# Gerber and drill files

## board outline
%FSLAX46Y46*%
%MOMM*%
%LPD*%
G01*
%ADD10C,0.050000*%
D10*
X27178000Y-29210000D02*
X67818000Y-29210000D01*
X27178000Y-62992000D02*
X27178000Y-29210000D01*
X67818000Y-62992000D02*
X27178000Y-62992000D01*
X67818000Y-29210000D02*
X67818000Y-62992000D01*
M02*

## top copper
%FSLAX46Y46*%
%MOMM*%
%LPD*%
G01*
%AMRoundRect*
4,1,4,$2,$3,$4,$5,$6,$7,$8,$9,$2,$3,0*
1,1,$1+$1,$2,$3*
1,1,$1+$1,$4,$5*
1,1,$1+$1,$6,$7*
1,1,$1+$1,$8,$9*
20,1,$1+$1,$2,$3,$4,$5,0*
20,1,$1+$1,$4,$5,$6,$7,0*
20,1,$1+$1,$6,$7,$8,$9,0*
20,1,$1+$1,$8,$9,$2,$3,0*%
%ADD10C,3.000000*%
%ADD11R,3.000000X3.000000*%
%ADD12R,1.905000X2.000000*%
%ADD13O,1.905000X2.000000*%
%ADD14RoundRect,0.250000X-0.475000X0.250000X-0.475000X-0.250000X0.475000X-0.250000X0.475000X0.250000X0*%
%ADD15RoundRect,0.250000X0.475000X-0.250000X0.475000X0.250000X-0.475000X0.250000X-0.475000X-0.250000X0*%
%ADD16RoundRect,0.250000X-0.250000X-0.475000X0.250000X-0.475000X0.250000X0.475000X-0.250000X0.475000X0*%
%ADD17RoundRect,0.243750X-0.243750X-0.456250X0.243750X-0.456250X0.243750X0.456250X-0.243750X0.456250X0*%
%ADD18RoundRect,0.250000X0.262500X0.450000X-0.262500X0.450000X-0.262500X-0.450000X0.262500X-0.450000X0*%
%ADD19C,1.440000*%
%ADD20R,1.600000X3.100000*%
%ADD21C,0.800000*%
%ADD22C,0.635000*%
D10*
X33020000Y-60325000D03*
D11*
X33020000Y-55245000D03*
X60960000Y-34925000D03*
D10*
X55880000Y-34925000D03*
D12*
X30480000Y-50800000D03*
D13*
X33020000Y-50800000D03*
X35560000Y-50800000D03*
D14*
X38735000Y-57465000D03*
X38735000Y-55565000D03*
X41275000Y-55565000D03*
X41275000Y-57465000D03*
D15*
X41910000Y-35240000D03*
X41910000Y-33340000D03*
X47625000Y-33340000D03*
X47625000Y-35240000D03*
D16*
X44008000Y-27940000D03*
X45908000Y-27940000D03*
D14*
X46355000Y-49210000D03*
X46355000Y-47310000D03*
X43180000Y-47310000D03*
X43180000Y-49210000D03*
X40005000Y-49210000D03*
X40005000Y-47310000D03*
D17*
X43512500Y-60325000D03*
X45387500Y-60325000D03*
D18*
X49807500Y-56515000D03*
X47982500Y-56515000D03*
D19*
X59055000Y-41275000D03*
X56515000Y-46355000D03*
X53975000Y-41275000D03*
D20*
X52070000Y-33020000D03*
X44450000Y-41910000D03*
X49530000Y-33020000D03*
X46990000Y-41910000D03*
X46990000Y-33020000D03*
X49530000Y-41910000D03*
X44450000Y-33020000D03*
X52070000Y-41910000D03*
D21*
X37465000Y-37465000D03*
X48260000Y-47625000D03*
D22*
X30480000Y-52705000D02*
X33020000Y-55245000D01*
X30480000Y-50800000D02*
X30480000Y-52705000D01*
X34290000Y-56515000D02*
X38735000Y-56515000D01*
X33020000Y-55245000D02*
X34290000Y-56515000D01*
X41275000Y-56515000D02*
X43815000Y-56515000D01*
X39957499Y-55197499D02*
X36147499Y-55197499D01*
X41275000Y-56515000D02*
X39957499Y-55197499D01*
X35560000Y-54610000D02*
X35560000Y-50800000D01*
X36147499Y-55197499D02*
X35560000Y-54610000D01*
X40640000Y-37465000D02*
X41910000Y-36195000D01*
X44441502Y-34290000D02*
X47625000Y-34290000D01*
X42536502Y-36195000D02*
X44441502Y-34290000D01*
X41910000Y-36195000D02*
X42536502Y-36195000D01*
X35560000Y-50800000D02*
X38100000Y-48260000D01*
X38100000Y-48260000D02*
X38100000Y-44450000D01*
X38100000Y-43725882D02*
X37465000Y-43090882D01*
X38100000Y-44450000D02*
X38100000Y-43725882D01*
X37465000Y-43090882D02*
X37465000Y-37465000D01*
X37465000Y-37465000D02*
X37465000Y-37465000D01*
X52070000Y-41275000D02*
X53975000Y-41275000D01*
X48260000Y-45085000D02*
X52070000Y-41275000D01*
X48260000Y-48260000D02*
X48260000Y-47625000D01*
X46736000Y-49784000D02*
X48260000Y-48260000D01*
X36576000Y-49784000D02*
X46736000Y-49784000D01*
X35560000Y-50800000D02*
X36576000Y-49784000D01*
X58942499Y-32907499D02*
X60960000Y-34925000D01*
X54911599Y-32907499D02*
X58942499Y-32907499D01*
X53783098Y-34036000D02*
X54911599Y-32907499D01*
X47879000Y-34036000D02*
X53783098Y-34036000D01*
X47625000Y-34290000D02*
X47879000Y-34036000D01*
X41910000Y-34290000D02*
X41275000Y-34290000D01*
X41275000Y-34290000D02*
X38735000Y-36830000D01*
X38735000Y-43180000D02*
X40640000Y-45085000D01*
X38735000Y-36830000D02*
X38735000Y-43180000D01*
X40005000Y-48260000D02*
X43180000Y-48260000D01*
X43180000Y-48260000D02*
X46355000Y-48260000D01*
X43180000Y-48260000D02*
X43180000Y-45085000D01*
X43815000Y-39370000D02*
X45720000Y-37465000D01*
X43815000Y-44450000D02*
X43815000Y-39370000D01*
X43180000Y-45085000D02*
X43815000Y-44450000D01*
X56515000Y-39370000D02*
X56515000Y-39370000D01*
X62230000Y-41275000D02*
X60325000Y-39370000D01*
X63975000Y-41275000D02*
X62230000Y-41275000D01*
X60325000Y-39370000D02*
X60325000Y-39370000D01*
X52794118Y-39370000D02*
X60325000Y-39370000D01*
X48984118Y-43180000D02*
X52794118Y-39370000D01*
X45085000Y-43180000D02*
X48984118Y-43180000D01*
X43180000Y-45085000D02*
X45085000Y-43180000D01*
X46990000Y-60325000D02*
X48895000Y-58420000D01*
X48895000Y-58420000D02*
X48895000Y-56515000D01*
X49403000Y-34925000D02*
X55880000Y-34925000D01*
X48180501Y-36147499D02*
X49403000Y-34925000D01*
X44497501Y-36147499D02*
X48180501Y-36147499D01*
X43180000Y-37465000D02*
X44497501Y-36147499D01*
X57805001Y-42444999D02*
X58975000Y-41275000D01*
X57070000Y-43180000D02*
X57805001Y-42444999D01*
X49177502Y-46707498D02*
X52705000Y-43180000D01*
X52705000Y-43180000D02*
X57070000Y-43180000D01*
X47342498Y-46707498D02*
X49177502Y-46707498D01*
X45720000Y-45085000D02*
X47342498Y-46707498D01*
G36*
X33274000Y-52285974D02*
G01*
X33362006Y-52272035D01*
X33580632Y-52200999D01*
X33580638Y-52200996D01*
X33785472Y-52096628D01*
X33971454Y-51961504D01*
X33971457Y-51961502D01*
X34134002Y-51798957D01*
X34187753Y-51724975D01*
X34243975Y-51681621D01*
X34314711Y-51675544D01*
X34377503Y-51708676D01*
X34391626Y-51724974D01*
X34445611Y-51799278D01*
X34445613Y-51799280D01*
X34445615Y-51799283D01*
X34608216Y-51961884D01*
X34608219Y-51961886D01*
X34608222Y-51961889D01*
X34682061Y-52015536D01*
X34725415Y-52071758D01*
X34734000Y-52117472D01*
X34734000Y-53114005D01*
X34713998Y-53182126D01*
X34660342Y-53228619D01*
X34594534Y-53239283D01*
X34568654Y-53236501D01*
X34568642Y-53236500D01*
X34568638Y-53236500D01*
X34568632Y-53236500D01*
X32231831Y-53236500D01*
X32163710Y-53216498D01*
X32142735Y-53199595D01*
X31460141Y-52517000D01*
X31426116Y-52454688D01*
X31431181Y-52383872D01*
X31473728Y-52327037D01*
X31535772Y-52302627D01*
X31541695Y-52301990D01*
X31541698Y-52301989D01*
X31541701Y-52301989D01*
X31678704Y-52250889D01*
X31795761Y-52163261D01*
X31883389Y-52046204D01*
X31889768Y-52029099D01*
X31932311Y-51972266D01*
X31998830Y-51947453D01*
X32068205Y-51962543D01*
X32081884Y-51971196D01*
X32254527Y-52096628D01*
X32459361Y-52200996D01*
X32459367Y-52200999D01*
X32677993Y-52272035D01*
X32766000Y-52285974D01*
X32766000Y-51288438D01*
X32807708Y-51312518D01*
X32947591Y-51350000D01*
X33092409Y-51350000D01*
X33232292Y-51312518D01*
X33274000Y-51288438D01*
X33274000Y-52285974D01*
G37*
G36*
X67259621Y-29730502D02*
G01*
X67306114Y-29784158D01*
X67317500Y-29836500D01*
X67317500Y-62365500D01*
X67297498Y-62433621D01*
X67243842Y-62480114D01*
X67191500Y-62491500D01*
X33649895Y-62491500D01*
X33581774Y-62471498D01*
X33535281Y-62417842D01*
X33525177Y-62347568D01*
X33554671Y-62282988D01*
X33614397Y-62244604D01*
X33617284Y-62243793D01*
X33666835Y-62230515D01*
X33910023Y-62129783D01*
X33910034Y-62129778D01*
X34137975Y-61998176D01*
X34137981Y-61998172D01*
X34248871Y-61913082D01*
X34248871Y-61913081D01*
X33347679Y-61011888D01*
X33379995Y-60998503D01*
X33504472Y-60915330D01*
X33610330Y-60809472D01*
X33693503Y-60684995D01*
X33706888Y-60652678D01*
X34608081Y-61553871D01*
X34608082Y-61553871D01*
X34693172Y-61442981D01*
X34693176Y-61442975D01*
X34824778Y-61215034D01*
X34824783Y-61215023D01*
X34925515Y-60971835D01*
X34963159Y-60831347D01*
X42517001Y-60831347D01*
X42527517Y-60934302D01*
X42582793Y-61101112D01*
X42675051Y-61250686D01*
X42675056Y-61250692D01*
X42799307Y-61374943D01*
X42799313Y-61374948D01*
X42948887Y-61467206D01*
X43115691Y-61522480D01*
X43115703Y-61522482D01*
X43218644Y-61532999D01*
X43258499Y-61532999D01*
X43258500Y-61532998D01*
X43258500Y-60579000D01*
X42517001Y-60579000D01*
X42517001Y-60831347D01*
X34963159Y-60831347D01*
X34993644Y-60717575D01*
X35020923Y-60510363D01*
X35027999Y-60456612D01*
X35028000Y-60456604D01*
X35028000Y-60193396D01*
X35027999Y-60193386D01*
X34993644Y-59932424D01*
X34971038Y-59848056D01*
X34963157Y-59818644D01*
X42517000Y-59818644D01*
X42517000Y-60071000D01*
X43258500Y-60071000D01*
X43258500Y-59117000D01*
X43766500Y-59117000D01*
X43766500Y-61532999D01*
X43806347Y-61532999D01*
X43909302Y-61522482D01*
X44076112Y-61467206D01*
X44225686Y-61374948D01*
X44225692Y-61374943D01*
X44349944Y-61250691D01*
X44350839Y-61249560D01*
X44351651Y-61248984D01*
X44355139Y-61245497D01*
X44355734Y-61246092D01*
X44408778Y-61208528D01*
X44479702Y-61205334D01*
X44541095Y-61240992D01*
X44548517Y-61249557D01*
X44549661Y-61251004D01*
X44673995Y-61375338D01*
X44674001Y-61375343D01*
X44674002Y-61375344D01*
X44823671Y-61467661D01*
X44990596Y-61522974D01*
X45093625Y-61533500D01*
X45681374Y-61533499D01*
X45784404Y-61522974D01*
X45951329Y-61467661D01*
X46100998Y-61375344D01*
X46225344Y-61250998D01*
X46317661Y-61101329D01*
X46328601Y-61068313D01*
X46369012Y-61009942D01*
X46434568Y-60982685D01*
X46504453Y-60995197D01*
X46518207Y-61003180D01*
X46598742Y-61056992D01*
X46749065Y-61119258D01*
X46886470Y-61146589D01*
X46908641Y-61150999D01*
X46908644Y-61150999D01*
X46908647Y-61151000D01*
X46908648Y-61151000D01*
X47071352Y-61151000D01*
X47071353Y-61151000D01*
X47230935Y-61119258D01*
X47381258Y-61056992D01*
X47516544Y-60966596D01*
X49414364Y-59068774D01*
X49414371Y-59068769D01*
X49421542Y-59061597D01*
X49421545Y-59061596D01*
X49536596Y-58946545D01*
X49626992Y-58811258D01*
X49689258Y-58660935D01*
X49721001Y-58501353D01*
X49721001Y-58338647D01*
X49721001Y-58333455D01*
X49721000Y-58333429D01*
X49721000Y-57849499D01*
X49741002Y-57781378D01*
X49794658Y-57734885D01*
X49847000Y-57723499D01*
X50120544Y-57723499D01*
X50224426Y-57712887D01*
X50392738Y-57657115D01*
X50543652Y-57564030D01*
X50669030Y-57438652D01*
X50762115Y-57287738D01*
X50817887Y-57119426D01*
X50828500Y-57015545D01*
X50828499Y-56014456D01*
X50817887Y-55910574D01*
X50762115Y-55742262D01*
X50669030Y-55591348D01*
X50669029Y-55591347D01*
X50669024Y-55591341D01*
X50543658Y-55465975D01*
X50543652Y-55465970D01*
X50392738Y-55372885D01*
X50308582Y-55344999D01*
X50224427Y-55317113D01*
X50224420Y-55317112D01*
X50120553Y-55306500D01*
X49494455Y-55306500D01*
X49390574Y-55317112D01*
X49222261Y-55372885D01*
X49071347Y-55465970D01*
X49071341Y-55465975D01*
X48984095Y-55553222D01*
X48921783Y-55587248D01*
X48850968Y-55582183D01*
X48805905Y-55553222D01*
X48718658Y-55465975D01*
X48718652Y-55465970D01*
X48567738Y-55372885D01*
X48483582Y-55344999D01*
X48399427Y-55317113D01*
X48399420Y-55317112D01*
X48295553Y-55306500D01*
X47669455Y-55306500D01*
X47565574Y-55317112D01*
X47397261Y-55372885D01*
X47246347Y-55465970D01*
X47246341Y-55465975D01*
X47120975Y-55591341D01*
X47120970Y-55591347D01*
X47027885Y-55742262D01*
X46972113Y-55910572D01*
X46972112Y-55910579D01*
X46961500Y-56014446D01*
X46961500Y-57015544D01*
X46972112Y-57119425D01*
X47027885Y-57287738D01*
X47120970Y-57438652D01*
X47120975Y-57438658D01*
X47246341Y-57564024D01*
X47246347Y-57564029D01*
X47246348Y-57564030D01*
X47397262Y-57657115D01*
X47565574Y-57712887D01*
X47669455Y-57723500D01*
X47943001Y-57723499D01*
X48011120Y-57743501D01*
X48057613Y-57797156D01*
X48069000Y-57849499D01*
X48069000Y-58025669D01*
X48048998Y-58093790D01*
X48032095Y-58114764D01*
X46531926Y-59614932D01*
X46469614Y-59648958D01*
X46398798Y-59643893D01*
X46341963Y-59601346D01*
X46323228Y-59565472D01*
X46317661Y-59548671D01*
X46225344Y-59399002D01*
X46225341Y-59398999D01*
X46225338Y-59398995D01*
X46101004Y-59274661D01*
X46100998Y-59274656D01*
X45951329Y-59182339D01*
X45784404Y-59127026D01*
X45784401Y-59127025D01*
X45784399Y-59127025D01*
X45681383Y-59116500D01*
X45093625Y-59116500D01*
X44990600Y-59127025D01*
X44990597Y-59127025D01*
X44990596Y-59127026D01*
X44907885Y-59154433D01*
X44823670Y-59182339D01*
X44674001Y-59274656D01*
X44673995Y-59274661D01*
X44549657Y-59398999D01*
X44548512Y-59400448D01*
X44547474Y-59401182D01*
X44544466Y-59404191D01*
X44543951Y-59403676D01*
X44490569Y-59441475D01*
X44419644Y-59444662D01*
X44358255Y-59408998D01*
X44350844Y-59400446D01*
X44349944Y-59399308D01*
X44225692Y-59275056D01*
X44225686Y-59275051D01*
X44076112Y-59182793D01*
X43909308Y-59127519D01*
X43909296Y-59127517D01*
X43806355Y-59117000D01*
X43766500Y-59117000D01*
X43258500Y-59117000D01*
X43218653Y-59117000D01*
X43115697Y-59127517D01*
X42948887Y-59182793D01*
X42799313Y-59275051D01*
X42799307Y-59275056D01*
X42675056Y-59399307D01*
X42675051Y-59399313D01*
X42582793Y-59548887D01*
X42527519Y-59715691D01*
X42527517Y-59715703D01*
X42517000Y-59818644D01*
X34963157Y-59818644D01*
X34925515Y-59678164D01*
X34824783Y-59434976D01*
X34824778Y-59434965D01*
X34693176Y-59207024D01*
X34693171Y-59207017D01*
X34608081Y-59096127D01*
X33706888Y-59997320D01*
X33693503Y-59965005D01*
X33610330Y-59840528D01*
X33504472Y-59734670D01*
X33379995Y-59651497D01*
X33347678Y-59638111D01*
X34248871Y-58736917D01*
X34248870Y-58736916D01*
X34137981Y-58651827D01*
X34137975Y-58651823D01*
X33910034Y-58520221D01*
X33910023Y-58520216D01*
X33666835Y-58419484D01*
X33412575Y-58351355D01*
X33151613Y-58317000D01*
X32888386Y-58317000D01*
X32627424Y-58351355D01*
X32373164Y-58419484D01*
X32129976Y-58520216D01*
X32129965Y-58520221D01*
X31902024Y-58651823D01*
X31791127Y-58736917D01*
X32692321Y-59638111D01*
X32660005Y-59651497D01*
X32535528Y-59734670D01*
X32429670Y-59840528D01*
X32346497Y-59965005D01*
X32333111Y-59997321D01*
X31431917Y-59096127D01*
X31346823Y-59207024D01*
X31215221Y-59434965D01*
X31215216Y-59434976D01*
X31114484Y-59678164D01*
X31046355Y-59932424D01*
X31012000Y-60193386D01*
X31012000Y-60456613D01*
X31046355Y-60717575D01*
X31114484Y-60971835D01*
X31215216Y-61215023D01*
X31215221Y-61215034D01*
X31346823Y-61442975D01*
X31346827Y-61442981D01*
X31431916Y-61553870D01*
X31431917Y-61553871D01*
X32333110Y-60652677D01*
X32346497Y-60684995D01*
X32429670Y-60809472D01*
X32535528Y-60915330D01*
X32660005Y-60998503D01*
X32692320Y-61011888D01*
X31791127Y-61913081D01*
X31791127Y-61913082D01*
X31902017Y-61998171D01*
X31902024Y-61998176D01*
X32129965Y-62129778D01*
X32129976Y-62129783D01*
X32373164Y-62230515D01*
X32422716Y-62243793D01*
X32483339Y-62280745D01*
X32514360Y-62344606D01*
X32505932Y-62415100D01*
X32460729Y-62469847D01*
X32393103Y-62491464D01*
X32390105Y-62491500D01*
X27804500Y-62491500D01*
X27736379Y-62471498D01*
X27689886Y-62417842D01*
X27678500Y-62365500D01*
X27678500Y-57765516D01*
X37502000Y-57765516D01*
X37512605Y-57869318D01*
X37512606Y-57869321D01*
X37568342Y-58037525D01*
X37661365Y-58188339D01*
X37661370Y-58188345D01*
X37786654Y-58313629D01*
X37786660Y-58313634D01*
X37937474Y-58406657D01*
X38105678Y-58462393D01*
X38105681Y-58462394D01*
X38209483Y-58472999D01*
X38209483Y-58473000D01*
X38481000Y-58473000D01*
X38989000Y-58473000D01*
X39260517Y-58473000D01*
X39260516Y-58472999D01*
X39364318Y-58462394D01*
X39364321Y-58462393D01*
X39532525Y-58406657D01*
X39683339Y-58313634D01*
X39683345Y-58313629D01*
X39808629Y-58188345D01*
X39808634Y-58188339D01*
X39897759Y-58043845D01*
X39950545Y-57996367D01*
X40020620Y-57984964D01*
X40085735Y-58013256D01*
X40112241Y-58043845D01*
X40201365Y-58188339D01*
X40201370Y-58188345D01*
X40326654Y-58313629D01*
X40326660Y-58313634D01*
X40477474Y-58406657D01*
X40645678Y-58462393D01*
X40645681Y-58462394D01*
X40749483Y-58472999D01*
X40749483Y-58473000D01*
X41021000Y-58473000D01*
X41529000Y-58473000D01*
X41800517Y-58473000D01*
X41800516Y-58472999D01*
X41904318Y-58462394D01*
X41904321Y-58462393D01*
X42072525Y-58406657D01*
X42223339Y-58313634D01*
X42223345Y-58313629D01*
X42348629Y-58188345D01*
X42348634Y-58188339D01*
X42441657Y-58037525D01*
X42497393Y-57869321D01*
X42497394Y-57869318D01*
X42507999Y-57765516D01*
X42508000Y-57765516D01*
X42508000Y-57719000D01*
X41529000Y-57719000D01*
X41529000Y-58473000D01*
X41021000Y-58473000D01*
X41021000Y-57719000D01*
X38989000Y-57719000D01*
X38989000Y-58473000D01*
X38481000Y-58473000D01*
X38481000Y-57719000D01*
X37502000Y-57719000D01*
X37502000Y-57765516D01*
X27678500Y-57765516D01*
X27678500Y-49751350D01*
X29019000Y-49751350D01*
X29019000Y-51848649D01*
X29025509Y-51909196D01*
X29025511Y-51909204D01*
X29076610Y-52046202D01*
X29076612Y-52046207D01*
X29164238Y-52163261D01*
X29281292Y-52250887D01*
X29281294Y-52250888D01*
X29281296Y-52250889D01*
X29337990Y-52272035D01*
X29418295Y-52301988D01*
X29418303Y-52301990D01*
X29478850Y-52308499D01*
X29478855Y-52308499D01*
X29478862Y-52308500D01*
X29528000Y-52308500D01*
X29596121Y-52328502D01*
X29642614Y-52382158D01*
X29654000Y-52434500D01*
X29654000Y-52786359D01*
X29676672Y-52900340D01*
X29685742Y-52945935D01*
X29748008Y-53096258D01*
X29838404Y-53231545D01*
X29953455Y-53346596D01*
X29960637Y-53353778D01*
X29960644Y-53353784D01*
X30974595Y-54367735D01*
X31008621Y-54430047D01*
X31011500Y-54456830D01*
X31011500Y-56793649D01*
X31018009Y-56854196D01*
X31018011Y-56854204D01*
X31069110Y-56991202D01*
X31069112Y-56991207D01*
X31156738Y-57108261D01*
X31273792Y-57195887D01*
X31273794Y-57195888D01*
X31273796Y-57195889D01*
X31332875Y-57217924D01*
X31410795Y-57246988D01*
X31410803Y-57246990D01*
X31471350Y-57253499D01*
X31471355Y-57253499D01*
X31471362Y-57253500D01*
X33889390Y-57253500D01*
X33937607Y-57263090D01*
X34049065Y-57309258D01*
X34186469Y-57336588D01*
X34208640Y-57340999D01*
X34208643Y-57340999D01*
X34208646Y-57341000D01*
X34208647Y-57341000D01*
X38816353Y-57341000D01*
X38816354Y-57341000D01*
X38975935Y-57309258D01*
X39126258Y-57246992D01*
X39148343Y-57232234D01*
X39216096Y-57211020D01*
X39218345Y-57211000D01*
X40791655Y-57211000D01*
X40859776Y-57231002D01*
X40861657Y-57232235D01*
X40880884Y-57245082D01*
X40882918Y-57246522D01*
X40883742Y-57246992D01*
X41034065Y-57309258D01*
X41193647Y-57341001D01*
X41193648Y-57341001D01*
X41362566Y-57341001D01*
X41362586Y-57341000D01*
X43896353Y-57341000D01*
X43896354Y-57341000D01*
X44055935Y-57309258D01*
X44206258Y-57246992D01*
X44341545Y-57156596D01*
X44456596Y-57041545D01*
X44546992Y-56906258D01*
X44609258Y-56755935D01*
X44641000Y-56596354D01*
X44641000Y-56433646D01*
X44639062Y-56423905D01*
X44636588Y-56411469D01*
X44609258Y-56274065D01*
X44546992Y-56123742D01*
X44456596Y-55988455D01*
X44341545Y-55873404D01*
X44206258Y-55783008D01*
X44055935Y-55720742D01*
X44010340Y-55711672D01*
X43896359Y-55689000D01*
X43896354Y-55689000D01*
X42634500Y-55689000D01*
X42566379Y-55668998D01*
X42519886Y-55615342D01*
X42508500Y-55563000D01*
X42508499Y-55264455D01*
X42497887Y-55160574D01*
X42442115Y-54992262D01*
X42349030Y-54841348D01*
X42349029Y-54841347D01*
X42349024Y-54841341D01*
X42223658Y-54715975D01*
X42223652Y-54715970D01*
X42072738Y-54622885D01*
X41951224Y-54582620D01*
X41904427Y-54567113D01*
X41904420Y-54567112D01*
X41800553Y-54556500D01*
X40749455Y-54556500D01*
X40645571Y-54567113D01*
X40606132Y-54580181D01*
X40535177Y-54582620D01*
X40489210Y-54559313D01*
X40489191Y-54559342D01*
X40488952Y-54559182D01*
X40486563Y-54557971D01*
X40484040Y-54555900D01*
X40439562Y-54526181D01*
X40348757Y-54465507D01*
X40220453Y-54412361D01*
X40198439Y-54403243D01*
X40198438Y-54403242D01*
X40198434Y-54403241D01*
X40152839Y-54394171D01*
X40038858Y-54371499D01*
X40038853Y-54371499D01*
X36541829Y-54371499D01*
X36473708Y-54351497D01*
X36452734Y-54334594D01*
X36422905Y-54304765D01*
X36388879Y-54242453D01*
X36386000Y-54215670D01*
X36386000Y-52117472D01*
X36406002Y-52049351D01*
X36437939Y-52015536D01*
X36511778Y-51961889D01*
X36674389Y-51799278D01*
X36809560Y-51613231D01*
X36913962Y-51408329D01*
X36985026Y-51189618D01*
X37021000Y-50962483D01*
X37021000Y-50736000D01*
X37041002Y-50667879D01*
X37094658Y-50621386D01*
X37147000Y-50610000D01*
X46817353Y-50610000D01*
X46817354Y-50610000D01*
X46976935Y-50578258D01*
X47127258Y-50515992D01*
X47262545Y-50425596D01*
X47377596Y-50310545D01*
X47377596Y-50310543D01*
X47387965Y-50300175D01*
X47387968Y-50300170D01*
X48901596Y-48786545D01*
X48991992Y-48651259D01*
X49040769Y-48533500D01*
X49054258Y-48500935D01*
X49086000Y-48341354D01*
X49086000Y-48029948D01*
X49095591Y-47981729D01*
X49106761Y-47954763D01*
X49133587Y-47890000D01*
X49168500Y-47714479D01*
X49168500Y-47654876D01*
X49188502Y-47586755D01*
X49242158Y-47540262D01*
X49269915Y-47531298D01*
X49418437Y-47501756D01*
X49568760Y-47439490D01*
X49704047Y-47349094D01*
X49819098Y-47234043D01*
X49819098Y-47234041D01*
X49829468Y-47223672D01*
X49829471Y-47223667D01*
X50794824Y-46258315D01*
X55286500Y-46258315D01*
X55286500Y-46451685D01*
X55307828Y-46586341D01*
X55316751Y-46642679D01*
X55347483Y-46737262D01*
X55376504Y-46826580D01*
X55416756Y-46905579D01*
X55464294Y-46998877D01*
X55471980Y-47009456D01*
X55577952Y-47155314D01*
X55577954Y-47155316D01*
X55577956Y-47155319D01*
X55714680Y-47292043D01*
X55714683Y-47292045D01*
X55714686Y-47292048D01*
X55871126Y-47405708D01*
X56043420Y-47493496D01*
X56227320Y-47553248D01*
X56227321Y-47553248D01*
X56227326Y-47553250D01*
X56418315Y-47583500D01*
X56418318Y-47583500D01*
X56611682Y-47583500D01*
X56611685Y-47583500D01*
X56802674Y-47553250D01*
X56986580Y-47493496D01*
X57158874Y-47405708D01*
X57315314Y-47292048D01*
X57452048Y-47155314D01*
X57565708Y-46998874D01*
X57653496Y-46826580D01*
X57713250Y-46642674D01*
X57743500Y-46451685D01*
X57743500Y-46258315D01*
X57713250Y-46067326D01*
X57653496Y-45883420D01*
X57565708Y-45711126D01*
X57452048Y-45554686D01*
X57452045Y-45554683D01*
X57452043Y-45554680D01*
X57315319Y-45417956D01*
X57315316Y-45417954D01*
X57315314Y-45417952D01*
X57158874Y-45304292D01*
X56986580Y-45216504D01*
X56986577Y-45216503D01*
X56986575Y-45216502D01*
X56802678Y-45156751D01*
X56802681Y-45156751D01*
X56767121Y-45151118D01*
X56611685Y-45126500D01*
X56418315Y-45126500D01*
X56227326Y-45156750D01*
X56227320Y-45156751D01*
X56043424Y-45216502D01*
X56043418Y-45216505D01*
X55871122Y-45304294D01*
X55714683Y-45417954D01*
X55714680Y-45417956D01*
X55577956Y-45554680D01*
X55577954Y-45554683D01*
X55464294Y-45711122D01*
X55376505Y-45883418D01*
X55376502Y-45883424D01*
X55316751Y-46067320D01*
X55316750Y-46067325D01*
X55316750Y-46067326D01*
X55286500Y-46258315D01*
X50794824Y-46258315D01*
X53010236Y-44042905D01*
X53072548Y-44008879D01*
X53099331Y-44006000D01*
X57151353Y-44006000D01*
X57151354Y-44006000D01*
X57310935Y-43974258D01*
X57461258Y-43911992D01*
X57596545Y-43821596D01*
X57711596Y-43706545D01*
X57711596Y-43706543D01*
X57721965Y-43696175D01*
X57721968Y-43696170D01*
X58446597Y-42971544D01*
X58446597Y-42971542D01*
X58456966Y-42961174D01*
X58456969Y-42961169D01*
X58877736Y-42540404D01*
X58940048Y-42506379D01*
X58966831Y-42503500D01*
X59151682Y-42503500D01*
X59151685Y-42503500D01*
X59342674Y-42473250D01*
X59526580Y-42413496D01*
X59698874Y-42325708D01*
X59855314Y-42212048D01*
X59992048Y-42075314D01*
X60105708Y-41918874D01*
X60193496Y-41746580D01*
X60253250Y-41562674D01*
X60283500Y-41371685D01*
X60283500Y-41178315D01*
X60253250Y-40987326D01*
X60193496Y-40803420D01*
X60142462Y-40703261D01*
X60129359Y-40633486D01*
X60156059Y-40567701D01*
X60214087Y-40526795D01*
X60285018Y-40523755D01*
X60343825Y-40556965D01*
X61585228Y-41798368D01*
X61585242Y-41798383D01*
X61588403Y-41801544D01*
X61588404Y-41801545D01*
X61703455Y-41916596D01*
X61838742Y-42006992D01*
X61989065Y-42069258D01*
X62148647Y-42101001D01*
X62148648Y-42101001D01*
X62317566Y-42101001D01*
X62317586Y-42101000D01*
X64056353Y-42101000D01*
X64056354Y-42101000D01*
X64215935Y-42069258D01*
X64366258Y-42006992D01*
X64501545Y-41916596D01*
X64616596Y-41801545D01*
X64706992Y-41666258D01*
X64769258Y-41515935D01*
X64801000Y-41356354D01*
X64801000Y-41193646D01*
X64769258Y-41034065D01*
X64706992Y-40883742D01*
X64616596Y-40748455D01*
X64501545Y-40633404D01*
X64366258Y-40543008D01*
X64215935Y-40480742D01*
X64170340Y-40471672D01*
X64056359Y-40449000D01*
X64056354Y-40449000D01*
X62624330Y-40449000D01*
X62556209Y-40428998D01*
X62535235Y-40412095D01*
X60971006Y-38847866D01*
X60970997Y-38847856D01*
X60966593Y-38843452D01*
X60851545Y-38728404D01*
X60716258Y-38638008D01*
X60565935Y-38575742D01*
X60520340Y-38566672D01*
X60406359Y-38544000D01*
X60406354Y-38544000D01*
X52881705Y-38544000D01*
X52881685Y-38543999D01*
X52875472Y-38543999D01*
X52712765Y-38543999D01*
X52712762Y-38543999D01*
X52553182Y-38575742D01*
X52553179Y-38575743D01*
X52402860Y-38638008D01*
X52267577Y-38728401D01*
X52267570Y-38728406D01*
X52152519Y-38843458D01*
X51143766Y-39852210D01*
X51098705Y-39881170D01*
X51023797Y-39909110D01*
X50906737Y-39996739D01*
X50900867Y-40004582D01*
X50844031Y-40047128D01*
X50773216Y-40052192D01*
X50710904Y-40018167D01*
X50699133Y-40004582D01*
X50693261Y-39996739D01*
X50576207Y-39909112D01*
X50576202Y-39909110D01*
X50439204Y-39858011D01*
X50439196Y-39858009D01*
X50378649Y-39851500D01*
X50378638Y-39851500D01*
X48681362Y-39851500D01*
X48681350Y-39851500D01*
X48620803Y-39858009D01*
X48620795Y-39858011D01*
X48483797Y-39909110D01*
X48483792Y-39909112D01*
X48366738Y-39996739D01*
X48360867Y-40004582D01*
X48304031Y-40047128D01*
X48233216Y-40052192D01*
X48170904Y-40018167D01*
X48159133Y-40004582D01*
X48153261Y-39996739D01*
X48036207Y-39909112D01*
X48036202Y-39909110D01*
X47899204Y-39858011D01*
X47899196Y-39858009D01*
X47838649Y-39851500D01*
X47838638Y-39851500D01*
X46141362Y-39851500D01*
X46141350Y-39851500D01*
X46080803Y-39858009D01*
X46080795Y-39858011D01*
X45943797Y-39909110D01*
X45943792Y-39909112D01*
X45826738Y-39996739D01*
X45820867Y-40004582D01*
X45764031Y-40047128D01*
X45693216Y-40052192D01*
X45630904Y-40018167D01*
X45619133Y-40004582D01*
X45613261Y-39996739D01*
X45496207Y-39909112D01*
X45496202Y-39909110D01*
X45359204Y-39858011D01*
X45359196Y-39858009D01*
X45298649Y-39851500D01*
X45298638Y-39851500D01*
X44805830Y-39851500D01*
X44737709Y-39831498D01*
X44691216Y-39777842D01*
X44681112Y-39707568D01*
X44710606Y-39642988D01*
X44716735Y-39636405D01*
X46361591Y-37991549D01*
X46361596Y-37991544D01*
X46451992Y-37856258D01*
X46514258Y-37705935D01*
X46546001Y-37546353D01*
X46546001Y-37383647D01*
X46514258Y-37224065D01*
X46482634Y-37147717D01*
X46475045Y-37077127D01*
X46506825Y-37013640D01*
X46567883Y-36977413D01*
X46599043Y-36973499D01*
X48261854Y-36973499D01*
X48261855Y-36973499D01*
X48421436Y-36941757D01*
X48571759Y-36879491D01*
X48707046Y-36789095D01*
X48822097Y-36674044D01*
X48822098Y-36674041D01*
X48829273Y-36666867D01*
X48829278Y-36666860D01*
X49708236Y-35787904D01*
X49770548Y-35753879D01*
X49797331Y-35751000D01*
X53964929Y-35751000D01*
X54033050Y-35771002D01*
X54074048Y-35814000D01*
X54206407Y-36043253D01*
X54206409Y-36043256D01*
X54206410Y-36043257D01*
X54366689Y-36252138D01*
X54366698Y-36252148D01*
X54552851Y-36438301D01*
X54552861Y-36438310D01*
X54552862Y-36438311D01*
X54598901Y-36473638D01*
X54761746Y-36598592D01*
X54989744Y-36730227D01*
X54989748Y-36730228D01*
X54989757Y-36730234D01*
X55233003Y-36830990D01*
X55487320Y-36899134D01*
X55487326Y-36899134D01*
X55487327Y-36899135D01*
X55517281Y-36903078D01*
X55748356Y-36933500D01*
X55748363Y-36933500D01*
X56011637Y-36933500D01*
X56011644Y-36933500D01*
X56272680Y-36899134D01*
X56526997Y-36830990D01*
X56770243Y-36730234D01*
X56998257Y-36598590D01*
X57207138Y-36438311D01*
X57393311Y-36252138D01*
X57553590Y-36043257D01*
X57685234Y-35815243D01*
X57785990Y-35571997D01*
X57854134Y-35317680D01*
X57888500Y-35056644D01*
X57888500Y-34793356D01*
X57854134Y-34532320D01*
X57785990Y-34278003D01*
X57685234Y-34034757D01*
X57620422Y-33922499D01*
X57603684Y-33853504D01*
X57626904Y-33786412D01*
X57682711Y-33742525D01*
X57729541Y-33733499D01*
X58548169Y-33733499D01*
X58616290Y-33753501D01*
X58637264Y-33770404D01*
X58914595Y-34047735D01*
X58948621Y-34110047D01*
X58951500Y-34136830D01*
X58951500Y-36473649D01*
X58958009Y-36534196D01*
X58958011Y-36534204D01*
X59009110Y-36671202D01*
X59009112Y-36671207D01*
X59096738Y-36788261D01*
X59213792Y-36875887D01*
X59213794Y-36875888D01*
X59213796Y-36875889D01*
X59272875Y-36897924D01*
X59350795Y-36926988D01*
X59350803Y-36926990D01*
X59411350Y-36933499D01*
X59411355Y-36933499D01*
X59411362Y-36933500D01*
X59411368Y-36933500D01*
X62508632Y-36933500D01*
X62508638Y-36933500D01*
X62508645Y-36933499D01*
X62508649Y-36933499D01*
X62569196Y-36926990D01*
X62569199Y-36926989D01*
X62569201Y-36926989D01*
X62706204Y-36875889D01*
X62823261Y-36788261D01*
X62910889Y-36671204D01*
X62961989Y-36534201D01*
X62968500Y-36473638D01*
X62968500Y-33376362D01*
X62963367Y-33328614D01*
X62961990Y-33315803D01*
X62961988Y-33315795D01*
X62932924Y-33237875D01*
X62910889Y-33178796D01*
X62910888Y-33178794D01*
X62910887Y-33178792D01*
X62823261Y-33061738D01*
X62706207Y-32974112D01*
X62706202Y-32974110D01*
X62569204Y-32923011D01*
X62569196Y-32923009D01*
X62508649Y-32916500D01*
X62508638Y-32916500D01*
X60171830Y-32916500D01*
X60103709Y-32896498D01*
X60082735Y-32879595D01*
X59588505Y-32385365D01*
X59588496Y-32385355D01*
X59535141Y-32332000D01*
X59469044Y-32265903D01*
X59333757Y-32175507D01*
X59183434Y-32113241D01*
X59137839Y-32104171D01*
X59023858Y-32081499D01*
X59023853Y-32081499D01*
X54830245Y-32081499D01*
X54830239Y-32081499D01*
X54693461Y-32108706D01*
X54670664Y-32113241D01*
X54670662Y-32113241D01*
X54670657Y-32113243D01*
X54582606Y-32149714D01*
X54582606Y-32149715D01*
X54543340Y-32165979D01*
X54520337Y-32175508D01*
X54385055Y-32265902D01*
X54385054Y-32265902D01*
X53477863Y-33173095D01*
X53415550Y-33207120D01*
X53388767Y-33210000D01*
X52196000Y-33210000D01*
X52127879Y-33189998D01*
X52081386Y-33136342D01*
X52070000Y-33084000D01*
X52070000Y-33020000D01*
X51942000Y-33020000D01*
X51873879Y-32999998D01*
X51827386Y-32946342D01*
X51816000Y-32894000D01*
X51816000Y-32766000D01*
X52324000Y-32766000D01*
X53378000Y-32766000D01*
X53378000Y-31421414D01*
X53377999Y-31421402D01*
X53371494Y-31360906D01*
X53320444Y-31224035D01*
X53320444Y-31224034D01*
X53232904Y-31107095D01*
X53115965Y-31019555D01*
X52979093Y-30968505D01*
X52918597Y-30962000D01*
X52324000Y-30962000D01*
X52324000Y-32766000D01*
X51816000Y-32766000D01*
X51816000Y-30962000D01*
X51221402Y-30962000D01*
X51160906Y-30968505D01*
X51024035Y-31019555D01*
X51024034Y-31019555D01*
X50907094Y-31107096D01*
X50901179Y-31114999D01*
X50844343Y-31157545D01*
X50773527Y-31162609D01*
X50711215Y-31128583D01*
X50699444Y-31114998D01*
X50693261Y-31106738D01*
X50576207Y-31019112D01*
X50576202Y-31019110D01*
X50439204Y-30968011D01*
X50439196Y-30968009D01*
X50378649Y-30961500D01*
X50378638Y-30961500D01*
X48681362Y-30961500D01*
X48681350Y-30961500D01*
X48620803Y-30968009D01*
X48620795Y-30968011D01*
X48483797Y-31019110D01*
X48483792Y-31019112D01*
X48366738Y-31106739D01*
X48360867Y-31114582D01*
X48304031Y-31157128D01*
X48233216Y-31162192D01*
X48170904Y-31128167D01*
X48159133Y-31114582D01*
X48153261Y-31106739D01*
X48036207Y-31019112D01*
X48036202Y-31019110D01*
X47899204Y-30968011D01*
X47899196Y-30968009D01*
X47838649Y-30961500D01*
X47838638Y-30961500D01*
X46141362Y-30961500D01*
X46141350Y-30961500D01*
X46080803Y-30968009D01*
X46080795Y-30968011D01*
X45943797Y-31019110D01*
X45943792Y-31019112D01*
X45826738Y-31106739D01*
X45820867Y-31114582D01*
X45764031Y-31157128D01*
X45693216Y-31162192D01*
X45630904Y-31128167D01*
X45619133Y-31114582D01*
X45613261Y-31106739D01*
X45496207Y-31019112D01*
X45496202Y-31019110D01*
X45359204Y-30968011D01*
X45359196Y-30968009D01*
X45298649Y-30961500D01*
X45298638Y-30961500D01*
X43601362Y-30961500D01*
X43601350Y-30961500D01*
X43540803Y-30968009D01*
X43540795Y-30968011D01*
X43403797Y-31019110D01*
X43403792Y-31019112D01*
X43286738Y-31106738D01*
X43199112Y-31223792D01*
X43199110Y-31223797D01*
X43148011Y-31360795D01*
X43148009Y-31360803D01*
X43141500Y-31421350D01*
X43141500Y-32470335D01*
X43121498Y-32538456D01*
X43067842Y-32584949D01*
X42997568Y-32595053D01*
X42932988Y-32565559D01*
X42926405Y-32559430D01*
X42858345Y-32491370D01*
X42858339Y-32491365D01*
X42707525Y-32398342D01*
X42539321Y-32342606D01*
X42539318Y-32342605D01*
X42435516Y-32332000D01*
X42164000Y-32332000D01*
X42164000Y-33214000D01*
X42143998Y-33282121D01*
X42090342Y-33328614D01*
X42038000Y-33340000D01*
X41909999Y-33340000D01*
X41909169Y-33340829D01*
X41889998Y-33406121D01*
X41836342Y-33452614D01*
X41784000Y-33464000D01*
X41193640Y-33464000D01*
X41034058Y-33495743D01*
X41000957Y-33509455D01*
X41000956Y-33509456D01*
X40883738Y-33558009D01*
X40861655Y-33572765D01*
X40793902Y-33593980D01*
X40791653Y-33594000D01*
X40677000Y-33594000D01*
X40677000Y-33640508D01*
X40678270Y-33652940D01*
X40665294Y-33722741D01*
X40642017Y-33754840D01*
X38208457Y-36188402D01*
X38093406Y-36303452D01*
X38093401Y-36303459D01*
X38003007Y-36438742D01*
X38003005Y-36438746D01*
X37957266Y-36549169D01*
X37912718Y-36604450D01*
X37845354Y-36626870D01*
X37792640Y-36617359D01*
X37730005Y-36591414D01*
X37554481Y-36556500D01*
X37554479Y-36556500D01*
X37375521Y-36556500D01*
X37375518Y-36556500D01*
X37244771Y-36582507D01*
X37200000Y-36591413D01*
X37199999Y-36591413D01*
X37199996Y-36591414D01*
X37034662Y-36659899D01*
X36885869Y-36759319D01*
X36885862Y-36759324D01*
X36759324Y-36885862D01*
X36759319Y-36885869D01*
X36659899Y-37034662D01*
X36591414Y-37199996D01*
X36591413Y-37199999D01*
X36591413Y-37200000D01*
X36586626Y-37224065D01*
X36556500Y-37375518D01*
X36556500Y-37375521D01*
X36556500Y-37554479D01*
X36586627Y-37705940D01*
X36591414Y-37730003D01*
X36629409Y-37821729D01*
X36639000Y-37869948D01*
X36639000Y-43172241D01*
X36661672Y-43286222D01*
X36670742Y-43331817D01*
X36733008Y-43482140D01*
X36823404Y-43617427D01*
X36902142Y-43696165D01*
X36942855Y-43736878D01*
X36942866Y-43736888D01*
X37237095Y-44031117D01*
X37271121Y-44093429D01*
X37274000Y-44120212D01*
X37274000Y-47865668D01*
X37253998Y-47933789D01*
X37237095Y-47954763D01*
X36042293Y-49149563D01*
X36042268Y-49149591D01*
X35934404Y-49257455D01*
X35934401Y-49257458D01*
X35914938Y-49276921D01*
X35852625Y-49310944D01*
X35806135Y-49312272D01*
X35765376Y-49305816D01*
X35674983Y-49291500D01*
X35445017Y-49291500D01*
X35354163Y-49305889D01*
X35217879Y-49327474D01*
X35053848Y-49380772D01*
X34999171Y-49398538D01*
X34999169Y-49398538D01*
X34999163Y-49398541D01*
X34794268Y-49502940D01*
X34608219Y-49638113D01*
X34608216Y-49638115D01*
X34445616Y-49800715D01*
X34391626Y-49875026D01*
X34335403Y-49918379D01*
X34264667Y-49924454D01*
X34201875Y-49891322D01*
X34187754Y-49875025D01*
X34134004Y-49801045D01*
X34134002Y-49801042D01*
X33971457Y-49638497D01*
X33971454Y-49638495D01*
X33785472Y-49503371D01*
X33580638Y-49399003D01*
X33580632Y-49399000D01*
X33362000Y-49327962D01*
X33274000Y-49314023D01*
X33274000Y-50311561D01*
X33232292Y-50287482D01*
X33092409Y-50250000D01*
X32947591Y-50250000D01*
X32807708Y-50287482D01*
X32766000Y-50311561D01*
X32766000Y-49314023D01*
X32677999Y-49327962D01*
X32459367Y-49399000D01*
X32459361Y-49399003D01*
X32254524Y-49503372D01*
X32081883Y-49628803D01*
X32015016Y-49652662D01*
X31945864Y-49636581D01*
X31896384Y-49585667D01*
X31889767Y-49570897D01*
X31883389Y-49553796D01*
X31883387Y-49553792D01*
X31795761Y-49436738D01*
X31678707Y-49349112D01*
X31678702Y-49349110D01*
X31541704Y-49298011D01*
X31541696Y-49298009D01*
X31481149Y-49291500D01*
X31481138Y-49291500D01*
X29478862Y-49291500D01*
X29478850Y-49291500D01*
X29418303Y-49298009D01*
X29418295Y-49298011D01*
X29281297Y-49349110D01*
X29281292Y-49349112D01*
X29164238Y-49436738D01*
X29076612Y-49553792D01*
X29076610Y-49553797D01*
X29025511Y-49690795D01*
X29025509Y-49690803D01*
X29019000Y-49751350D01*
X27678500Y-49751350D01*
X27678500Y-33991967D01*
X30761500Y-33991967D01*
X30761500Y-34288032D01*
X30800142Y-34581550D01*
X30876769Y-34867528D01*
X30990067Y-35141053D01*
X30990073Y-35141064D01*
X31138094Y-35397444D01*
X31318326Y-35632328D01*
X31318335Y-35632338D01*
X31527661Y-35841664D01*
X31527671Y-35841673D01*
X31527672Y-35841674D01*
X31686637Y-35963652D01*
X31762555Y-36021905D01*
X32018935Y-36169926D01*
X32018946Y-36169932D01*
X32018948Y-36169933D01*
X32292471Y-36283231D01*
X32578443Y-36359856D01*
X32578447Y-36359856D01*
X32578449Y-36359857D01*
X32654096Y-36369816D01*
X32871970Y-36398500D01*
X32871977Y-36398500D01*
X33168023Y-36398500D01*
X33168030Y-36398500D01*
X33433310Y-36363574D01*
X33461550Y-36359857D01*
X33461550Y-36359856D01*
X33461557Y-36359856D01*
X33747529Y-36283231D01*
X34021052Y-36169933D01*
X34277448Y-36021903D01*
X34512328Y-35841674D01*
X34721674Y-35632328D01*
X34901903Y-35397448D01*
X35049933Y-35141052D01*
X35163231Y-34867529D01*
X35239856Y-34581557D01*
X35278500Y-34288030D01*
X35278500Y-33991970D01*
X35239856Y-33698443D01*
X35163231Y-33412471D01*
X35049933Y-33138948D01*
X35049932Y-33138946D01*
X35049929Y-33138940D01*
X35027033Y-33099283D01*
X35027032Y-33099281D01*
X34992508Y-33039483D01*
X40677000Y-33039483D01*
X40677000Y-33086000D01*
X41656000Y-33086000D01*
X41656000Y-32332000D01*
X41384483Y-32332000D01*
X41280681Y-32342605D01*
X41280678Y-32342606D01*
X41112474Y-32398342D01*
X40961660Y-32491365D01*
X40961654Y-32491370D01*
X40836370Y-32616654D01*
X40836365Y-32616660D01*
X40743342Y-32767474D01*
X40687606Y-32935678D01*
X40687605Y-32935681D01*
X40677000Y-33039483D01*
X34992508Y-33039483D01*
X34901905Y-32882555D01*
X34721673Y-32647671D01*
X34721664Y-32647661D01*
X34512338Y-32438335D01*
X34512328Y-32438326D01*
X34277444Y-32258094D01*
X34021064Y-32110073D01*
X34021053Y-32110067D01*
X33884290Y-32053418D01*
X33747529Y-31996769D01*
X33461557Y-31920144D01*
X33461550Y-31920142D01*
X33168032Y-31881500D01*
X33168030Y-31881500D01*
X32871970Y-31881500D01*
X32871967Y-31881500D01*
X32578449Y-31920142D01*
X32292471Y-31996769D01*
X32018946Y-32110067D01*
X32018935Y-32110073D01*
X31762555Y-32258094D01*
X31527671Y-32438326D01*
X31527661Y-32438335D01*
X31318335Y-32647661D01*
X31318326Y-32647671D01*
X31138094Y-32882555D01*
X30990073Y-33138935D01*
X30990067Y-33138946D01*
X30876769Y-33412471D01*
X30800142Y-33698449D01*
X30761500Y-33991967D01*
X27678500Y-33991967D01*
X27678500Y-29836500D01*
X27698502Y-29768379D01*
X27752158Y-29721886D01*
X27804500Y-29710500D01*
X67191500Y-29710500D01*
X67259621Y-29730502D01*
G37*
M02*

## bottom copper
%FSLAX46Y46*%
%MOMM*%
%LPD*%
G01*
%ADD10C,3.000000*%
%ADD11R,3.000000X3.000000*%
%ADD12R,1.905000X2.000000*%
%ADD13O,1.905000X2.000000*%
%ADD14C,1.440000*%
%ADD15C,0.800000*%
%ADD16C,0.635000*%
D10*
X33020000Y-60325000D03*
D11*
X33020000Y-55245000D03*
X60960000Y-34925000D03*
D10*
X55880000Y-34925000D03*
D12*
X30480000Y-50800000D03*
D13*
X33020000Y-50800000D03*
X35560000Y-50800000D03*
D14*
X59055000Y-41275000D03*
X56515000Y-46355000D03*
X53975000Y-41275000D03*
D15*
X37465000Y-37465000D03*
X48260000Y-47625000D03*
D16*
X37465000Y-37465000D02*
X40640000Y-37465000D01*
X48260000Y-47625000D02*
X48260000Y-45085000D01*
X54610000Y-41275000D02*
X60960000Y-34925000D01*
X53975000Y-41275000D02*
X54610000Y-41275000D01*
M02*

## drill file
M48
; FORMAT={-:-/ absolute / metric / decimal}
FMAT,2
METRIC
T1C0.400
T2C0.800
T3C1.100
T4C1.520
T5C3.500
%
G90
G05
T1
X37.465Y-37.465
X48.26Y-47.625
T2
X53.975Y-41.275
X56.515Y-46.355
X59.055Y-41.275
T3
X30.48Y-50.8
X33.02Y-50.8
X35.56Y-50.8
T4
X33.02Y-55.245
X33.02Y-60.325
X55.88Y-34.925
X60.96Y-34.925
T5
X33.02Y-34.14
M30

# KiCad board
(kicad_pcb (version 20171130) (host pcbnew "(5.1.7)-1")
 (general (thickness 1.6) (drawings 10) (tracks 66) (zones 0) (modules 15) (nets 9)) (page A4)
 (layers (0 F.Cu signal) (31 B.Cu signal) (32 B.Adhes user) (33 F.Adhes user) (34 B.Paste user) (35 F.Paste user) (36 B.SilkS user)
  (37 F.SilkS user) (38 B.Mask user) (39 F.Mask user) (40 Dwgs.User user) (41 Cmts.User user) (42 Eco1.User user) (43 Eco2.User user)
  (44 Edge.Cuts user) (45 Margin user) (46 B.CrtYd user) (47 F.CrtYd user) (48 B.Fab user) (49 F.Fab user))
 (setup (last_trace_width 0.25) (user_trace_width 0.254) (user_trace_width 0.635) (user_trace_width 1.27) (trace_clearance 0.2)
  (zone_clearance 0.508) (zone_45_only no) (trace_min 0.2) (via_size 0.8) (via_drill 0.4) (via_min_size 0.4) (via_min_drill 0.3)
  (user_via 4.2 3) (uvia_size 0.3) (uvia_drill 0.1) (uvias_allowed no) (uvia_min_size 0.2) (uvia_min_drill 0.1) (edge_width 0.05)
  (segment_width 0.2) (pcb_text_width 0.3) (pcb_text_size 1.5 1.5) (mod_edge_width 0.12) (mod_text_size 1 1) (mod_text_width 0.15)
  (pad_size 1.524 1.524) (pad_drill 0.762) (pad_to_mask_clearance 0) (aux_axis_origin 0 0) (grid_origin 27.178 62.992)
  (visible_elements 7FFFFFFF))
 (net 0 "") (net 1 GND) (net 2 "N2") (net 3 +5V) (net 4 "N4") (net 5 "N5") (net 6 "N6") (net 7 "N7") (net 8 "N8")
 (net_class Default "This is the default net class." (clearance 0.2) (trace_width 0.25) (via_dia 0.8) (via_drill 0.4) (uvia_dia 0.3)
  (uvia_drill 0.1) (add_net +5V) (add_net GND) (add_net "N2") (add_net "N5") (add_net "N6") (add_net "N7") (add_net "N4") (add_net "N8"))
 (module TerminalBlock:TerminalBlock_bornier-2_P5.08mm (layer F.Cu) (at 33.02 55.245 270)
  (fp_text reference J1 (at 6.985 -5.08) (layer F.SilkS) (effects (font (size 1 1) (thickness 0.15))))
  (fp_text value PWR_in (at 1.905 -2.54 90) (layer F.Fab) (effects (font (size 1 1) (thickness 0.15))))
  (pad 2 thru_hole circle (at 5.08 0 270) (size 3 3) (drill 1.52) (layers *.Cu *.Mask) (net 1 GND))
  (pad 1 thru_hole rect (at 0 0 270) (size 3 3) (drill 1.52) (layers *.Cu *.Mask) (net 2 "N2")))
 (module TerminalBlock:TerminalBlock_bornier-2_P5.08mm (layer F.Cu) (at 60.96 34.925 180)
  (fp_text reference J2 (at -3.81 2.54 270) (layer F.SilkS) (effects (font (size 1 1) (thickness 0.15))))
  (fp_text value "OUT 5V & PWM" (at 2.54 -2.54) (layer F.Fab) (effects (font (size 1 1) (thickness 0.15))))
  (pad 1 thru_hole rect (at 0 0 180) (size 3 3) (drill 1.52) (layers *.Cu *.Mask) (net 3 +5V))
  (pad 2 thru_hole circle (at 5.08 0 180) (size 3 3) (drill 1.52) (layers *.Cu *.Mask) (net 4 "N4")))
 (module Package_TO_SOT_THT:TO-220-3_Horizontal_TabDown (layer F.Cu) (at 30.48 50.8)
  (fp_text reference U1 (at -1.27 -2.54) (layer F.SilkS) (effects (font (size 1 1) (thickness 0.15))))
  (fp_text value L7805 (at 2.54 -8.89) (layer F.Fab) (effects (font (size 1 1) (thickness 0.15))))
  (pad "" np_thru_hole oval (at 2.54 -16.66) (size 3.5 3.5) (drill 3.5) (layers *.Cu *.Mask))
  (pad 1 thru_hole rect (at 0 0) (size 1.905 2) (drill 1.1) (layers *.Cu *.Mask) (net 2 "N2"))
  (pad 2 thru_hole oval (at 2.54 0) (size 1.905 2) (drill 1.1) (layers *.Cu *.Mask) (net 1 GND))
  (pad 3 thru_hole oval (at 5.08 0) (size 1.905 2) (drill 1.1) (layers *.Cu *.Mask) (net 3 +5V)))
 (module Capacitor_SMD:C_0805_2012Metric (layer F.Cu) (at 38.735 56.515 270)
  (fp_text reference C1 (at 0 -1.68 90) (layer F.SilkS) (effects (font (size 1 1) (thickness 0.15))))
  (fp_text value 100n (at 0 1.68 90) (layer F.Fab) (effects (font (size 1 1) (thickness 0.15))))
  (pad 2 smd roundrect (at 0.95 0 270) (size 1 1.45) (layers F.Cu F.Paste F.Mask) (roundrect_rratio 0.25) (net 1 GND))
  (pad 1 smd roundrect (at -0.95 0 270) (size 1 1.45) (layers F.Cu F.Paste F.Mask) (roundrect_rratio 0.25) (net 2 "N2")))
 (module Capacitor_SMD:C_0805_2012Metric (layer F.Cu) (at 41.275 56.515 270)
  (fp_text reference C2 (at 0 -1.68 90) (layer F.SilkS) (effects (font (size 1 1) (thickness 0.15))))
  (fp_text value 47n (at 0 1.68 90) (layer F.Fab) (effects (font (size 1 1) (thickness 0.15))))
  (pad 1 smd roundrect (at -0.95 0 270) (size 1 1.45) (layers F.Cu F.Paste F.Mask) (roundrect_rratio 0.25) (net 3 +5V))
  (pad 2 smd roundrect (at 0.95 0 270) (size 1 1.45) (layers F.Cu F.Paste F.Mask) (roundrect_rratio 0.25) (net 1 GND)))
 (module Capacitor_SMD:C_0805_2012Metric (layer F.Cu) (at 41.91 34.29 90)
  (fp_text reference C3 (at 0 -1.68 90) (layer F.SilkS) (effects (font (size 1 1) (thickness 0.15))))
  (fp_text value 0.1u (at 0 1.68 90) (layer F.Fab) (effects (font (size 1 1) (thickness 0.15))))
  (pad 1 smd roundrect (at -0.95 0 90) (size 1 1.45) (layers F.Cu F.Paste F.Mask) (roundrect_rratio 0.25) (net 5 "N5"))
  (pad 2 smd roundrect (at 0.95 0 90) (size 1 1.45) (layers F.Cu F.Paste F.Mask) (roundrect_rratio 0.25) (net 1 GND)))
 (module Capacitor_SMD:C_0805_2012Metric (layer F.Cu) (at 47.625 34.29 90)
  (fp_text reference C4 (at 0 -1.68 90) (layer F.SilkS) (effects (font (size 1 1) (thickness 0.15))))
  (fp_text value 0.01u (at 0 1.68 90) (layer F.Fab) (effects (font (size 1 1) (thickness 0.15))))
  (pad 2 smd roundrect (at 0.95 0 90) (size 1 1.45) (layers F.Cu F.Paste F.Mask) (roundrect_rratio 0.25) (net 1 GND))
  (pad 1 smd roundrect (at -0.95 0 90) (size 1 1.45) (layers F.Cu F.Paste F.Mask) (roundrect_rratio 0.25) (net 3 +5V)))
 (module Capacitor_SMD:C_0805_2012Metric (layer F.Cu) (at 44.958 27.94)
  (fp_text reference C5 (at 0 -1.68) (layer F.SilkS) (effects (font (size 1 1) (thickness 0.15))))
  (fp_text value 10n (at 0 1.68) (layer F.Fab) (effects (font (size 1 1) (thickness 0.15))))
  (pad 1 smd roundrect (at -0.95 0) (size 1 1.45) (layers F.Cu F.Paste F.Mask) (roundrect_rratio 0.25) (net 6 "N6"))
  (pad 2 smd roundrect (at 0.95 0) (size 1 1.45) (layers F.Cu F.Paste F.Mask) (roundrect_rratio 0.25) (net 1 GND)))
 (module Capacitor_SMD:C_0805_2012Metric (layer F.Cu) (at 46.355 48.26 270)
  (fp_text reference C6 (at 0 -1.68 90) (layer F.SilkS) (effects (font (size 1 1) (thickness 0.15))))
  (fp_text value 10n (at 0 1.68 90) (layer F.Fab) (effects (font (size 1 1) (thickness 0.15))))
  (pad 2 smd roundrect (at 0.95 0 270) (size 1 1.45) (layers F.Cu F.Paste F.Mask) (roundrect_rratio 0.25) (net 1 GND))
  (pad 1 smd roundrect (at -0.95 0 270) (size 1 1.45) (layers F.Cu F.Paste F.Mask) (roundrect_rratio 0.25) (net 6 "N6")))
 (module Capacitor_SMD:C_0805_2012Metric (layer F.Cu) (at 43.18 48.26 270)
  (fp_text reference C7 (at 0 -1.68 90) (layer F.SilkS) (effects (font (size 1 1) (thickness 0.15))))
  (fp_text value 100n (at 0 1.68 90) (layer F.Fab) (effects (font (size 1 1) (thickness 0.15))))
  (pad 1 smd roundrect (at -0.95 0 270) (size 1 1.45) (layers F.Cu F.Paste F.Mask) (roundrect_rratio 0.25) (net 6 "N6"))
  (pad 2 smd roundrect (at 0.95 0 270) (size 1 1.45) (layers F.Cu F.Paste F.Mask) (roundrect_rratio 0.25) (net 1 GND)))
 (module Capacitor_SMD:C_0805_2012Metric (layer F.Cu) (at 40.005 48.26 270)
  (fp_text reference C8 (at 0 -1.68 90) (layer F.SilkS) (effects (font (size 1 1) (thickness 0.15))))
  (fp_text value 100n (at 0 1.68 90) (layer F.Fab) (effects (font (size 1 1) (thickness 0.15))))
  (pad 2 smd roundrect (at 0.95 0 270) (size 1 1.45) (layers F.Cu F.Paste F.Mask) (roundrect_rratio 0.25) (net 1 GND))
  (pad 1 smd roundrect (at -0.95 0 270) (size 1 1.45) (layers F.Cu F.Paste F.Mask) (roundrect_rratio 0.25) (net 6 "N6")))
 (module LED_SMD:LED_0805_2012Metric (layer F.Cu) (at 44.45 60.325)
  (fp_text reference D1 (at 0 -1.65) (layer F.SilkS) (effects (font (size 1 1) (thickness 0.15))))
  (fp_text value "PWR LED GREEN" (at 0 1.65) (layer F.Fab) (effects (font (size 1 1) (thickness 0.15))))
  (pad 1 smd roundrect (at -0.9375 0) (size 0.975 1.4) (layers F.Cu F.Paste F.Mask) (roundrect_rratio 0.25) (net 1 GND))
  (pad 2 smd roundrect (at 0.9375 0) (size 0.975 1.4) (layers F.Cu F.Paste F.Mask) (roundrect_rratio 0.25) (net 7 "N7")))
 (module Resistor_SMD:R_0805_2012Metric (layer F.Cu) (at 48.895 56.515 180)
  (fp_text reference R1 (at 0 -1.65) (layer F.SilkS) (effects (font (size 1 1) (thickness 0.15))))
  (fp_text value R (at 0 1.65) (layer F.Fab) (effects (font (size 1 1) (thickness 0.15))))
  (pad 1 smd roundrect (at -0.9125 0 180) (size 1.025 1.4) (layers F.Cu F.Paste F.Mask) (roundrect_rratio 0.243902) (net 7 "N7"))
  (pad 2 smd roundrect (at 0.9125 0 180) (size 1.025 1.4) (layers F.Cu F.Paste F.Mask) (roundrect_rratio 0.243902) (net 3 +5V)))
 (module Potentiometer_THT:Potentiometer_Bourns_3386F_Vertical (layer F.Cu) (at 53.975 41.275 270)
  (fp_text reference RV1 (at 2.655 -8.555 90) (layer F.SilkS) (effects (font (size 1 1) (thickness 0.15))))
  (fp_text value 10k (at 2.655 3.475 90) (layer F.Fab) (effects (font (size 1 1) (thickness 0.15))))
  (pad 3 thru_hole circle (at 0 -5.08 270) (size 1.44 1.44) (drill 0.8) (layers *.Cu *.Mask) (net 6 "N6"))
  (pad 2 thru_hole circle (at 5.08 -2.54 270) (size 1.44 1.44) (drill 0.8) (layers *.Cu *.Mask) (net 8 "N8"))
  (pad 1 thru_hole circle (at 0 0 270) (size 1.44 1.44) (drill 0.8) (layers *.Cu *.Mask) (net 3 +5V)))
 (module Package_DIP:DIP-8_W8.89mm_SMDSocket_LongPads (layer F.Cu) (at 48.26 37.465 270)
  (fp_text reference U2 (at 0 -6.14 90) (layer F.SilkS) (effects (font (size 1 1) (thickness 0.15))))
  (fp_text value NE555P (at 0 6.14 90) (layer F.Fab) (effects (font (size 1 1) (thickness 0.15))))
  (pad 1 smd rect (at -4.445 -3.81 270) (size 3.1 1.6) (layers F.Cu F.Paste F.Mask) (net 1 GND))
  (pad 5 smd rect (at 4.445 3.81 270) (size 3.1 1.6) (layers F.Cu F.Paste F.Mask) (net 5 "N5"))
  (pad 2 smd rect (at -4.445 -1.27 270) (size 3.1 1.6) (layers F.Cu F.Paste F.Mask) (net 6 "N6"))
  (pad 6 smd rect (at 4.445 1.27 270) (size 3.1 1.6) (layers F.Cu F.Paste F.Mask) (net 6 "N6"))
  (pad 3 smd rect (at -4.445 1.27 270) (size 3.1 1.6) (layers F.Cu F.Paste F.Mask) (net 4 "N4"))
  (pad 7 smd rect (at 4.445 -1.27 270) (size 3.1 1.6) (layers F.Cu F.Paste F.Mask) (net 8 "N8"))
  (pad 4 smd rect (at -4.445 3.81 270) (size 3.1 1.6) (layers F.Cu F.Paste F.Mask) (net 3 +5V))
  (pad 8 smd rect (at 4.445 -3.81 270) (size 3.1 1.6) (layers F.Cu F.Paste F.Mask) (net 3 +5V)))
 (gr_line (start 27.178 29.21) (end 67.818 29.21) (layer Edge.Cuts) (width 0.05))
 (gr_line (start 27.178 62.992) (end 27.178 29.21) (layer Edge.Cuts) (width 0.05))
 (gr_line (start 67.818 62.992) (end 27.178 62.992) (layer Edge.Cuts) (width 0.05))
 (gr_line (start 67.818 29.21) (end 67.818 62.992) (layer Edge.Cuts) (width 0.05))
 (segment (start 30.48 52.705) (end 33.02 55.245) (width 0.635) (layer F.Cu) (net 2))
 (segment (start 30.48 50.8) (end 30.48 52.705) (width 0.635) (layer F.Cu) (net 2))
 (segment (start 34.29 56.515) (end 38.735 56.515) (width 0.635) (layer F.Cu) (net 2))
 (segment (start 33.02 55.245) (end 34.29 56.515) (width 0.635) (layer F.Cu) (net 2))
 (segment (start 41.275 56.515) (end 43.815 56.515) (width 0.635) (layer F.Cu) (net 3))
 (segment (start 39.957499 55.197499) (end 36.147499 55.197499) (width 0.635) (layer F.Cu) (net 3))
 (segment (start 41.275 56.515) (end 39.957499 55.197499) (width 0.635) (layer F.Cu) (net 3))
 (segment (start 35.56 54.61) (end 35.56 50.8) (width 0.635) (layer F.Cu) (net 3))
 (segment (start 36.147499 55.197499) (end 35.56 54.61) (width 0.635) (layer F.Cu) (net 3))
 (segment (start 40.64 37.465) (end 41.91 36.195) (width 0.635) (layer F.Cu) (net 3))
 (segment (start 44.441502 34.29) (end 47.625 34.29) (width 0.635) (layer F.Cu) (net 3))
 (segment (start 42.536502 36.195) (end 44.441502 34.29) (width 0.635) (layer F.Cu) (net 3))
 (segment (start 41.91 36.195) (end 42.536502 36.195) (width 0.635) (layer F.Cu) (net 3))
 (segment (start 35.56 50.8) (end 38.1 48.26) (width 0.635) (layer F.Cu) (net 3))
 (segment (start 38.1 48.26) (end 38.1 44.45) (width 0.635) (layer F.Cu) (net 3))
 (segment (start 38.1 43.725882) (end 37.465 43.090882) (width 0.635) (layer F.Cu) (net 3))
 (segment (start 38.1 44.45) (end 38.1 43.725882) (width 0.635) (layer F.Cu) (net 3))
 (segment (start 37.465 43.090882) (end 37.465 37.465) (width 0.635) (layer F.Cu) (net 3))
 (segment (start 37.465 37.465) (end 37.465 37.465) (width 0.635) (layer F.Cu) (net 3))
 (via (at 37.465 37.465) (size 0.8) (drill 0.4) (layers F.Cu B.Cu) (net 3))
 (segment (start 37.465 37.465) (end 40.64 37.465) (width 0.635) (layer B.Cu) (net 3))
 (via (at 48.26 47.625) (size 0.8) (drill 0.4) (layers F.Cu B.Cu) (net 3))
 (segment (start 52.07 41.275) (end 53.975 41.275) (width 0.635) (layer F.Cu) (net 3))
 (segment (start 48.26 45.085) (end 52.07 41.275) (width 0.635) (layer F.Cu) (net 3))
 (segment (start 48.26 48.26) (end 48.26 47.625) (width 0.635) (layer F.Cu) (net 3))
 (segment (start 46.736 49.784) (end 48.26 48.26) (width 0.635) (layer F.Cu) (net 3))
 (segment (start 36.576 49.784) (end 46.736 49.784) (width 0.635) (layer F.Cu) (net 3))
 (segment (start 35.56 50.8) (end 36.576 49.784) (width 0.635) (layer F.Cu) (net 3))
 (segment (start 48.26 47.625) (end 48.26 45.085) (width 0.635) (layer B.Cu) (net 3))
 (segment (start 54.61 41.275) (end 60.96 34.925) (width 0.635) (layer B.Cu) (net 3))
 (segment (start 53.975 41.275) (end 54.61 41.275) (width 0.635) (layer B.Cu) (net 3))
 (segment (start 58.942499 32.907499) (end 60.96 34.925) (width 0.635) (layer F.Cu) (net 3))
 (segment (start 54.911599 32.907499) (end 58.942499 32.907499) (width 0.635) (layer F.Cu) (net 3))
 (segment (start 53.783098 34.036) (end 54.911599 32.907499) (width 0.635) (layer F.Cu) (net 3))
 (segment (start 47.879 34.036) (end 53.783098 34.036) (width 0.635) (layer F.Cu) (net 3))
 (segment (start 47.625 34.29) (end 47.879 34.036) (width 0.635) (layer F.Cu) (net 3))
 (segment (start 41.91 34.29) (end 41.275 34.29) (width 0.635) (layer F.Cu) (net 5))
 (segment (start 41.275 34.29) (end 38.735 36.83) (width 0.635) (layer F.Cu) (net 5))
 (segment (start 38.735 43.18) (end 40.64 45.085) (width 0.635) (layer F.Cu) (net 5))
 (segment (start 38.735 36.83) (end 38.735 43.18) (width 0.635) (layer F.Cu) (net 5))
 (segment (start 40.005 48.26) (end 43.18 48.26) (width 0.635) (layer F.Cu) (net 6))
 (segment (start 43.18 48.26) (end 46.355 48.26) (width 0.635) (layer F.Cu) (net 6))
 (segment (start 43.18 48.26) (end 43.18 45.085) (width 0.635) (layer F.Cu) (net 6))
 (segment (start 43.815 39.37) (end 45.72 37.465) (width 0.635) (layer F.Cu) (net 6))
 (segment (start 43.815 44.45) (end 43.815 39.37) (width 0.635) (layer F.Cu) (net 6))
 (segment (start 43.18 45.085) (end 43.815 44.45) (width 0.635) (layer F.Cu) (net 6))
 (segment (start 56.515 39.37) (end 56.515 39.37) (width 0.635) (layer F.Cu) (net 6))
 (segment (start 62.23 41.275) (end 60.325 39.37) (width 0.635) (layer F.Cu) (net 6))
 (segment (start 63.975 41.275) (end 62.23 41.275) (width 0.635) (layer F.Cu) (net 6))
 (segment (start 60.325 39.37) (end 60.325 39.37) (width 0.635) (layer F.Cu) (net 6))
 (segment (start 52.794118 39.37) (end 60.325 39.37) (width 0.635) (layer F.Cu) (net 6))
 (segment (start 48.984118 43.18) (end 52.794118 39.37) (width 0.635) (layer F.Cu) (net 6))
 (segment (start 45.085 43.18) (end 48.984118 43.18) (width 0.635) (layer F.Cu) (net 6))
 (segment (start 43.18 45.085) (end 45.085 43.18) (width 0.635) (layer F.Cu) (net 6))
 (segment (start 46.99 60.325) (end 48.895 58.42) (width 0.635) (layer F.Cu) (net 7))
 (segment (start 48.895 58.42) (end 48.895 56.515) (width 0.635) (layer F.Cu) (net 7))
 (segment (start 49.403 34.925) (end 55.88 34.925) (width 0.635) (layer F.Cu) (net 4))
 (segment (start 48.180501 36.147499) (end 49.403 34.925) (width 0.635) (layer F.Cu) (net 4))
 (segment (start 44.497501 36.147499) (end 48.180501 36.147499) (width 0.635) (layer F.Cu) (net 4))
 (segment (start 43.18 37.465) (end 44.497501 36.147499) (width 0.635) (layer F.Cu) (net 4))
 (segment (start 57.805001 42.444999) (end 58.975 41.275) (width 0.635) (layer F.Cu) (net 8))
 (segment (start 57.07 43.18) (end 57.805001 42.444999) (width 0.635) (layer F.Cu) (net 8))
 (segment (start 49.177502 46.707498) (end 52.705 43.18) (width 0.635) (layer F.Cu) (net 8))
 (segment (start 52.705 43.18) (end 57.07 43.18) (width 0.635) (layer F.Cu) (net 8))
 (segment (start 47.342498 46.707498) (end 49.177502 46.707498) (width 0.635) (layer F.Cu) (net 8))
 (segment (start 45.72 45.085) (end 47.342498 46.707498) (width 0.635) (layer F.Cu) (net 8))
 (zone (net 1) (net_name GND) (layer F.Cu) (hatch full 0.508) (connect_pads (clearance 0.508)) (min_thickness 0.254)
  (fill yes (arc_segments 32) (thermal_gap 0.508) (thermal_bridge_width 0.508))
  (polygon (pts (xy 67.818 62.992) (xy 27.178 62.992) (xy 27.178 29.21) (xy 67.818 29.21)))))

